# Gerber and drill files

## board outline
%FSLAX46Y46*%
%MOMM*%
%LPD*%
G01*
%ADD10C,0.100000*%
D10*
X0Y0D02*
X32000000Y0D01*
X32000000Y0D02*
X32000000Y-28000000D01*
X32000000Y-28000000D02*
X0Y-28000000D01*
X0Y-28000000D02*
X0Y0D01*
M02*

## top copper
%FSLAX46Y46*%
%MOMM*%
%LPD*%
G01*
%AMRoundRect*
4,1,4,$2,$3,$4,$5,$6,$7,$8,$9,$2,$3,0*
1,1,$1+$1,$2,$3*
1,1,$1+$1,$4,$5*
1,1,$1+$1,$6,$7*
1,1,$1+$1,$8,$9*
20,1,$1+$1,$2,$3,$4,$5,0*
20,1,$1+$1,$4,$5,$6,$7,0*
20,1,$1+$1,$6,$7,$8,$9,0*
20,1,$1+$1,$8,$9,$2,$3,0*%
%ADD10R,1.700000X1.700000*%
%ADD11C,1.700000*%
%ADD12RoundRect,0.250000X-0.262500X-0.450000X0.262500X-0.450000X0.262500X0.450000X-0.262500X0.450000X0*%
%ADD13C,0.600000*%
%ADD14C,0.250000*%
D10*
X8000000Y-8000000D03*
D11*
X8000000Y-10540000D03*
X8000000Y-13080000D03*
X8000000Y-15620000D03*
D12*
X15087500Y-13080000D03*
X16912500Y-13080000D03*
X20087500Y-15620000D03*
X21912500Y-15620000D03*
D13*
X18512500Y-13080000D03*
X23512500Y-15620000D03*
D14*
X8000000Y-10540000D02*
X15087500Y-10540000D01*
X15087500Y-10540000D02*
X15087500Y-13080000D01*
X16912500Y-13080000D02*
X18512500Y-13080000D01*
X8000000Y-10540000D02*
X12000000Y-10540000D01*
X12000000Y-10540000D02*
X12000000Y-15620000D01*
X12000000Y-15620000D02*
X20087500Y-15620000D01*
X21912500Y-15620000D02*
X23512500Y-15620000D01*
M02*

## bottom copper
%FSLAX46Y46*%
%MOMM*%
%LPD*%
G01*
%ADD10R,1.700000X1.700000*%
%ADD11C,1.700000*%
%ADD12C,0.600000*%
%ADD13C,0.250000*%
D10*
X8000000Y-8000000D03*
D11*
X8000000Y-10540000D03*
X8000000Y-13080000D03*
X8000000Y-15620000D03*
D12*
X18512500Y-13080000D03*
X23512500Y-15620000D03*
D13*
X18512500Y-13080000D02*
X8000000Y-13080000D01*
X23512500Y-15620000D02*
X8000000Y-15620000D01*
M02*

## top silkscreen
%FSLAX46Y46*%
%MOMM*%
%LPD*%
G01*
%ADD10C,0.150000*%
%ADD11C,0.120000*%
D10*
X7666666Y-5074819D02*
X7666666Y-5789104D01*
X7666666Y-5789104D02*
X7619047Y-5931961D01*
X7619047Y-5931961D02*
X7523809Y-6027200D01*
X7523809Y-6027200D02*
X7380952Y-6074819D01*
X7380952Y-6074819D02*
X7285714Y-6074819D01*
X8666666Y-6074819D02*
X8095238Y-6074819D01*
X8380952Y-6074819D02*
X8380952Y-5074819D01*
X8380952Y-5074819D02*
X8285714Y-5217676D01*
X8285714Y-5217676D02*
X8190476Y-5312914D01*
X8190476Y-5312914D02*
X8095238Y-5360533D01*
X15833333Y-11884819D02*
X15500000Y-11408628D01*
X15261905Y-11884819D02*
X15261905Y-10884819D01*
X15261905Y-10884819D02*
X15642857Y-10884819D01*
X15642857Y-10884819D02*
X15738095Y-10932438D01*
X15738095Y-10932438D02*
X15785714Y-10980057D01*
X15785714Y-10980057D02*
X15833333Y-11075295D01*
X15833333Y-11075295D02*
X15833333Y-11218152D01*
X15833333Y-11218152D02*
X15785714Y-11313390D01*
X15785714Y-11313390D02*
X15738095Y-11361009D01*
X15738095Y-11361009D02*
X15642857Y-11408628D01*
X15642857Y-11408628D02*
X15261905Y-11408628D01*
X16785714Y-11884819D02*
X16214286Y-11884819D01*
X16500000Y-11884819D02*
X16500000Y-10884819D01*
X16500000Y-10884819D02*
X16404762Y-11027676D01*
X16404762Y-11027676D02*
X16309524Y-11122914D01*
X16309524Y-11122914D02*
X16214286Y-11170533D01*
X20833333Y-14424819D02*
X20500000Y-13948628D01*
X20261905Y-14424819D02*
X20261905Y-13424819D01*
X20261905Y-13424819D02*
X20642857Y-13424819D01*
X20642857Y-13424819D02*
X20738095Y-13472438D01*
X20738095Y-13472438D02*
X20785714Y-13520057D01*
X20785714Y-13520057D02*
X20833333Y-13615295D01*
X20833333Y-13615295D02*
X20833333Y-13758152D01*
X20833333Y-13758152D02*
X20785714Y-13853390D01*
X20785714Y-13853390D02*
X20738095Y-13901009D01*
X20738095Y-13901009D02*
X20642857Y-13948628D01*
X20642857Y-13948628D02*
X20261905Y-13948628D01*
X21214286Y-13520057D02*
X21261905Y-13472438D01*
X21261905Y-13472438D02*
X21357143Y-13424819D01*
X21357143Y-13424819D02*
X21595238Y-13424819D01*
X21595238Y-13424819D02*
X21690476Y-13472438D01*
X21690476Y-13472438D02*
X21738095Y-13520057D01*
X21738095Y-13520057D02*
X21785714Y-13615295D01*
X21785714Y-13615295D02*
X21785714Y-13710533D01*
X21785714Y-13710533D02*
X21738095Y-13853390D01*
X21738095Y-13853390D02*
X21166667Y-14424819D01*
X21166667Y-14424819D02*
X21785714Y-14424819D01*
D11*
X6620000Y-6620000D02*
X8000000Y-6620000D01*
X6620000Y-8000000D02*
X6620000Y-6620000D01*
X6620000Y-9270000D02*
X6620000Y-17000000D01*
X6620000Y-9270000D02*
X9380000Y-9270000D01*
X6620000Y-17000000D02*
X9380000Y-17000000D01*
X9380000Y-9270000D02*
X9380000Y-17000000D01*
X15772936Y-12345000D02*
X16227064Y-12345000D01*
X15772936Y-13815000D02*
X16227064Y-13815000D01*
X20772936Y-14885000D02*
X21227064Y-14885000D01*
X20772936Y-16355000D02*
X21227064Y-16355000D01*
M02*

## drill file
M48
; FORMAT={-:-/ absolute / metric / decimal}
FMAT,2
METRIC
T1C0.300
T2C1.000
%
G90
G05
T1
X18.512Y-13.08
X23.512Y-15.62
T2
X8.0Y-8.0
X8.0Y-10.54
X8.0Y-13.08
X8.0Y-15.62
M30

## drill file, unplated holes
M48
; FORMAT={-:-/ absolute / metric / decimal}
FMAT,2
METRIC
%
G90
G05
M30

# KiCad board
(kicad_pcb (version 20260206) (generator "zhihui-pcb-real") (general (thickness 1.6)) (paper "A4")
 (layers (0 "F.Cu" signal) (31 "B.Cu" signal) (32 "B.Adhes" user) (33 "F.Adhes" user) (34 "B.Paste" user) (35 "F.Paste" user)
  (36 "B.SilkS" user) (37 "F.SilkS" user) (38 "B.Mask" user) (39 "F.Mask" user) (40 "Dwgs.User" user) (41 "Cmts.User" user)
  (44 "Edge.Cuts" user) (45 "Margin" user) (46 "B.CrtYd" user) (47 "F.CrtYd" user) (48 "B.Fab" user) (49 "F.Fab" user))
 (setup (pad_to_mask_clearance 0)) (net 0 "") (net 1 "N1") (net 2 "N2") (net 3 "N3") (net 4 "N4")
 (gr_line (start 0 0) (end 32 0) (stroke (width 0.1) (type default)) (layer "Edge.Cuts"))
 (gr_line (start 32 0) (end 32 28) (stroke (width 0.1) (type default)) (layer "Edge.Cuts"))
 (gr_line (start 32 28) (end 0 28) (stroke (width 0.1) (type default)) (layer "Edge.Cuts"))
 (gr_line (start 0 28) (end 0 0) (stroke (width 0.1) (type default)) (layer "Edge.Cuts"))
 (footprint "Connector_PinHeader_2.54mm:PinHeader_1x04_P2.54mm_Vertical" (layer "F.Cu")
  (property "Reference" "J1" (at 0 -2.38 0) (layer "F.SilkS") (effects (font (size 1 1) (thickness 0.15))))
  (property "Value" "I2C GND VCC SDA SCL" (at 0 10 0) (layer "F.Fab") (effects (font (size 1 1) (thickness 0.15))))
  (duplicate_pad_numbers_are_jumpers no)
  (fp_line (start -1.38 -1.38) (end 0 -1.38) (stroke (width 0.12) (type solid)) (layer "F.SilkS"))
  (fp_line (start -1.38 0) (end -1.38 -1.38) (stroke (width 0.12) (type solid)) (layer "F.SilkS"))
  (fp_line (start -1.38 1.27) (end -1.38 9) (stroke (width 0.12) (type solid)) (layer "F.SilkS"))
  (fp_line (start -1.38 1.27) (end 1.38 1.27) (stroke (width 0.12) (type solid)) (layer "F.SilkS"))
  (fp_line (start -1.38 9) (end 1.38 9) (stroke (width 0.12) (type solid)) (layer "F.SilkS"))
  (fp_line (start 1.38 1.27) (end 1.38 9) (stroke (width 0.12) (type solid)) (layer "F.SilkS"))
  (pad "1" thru_hole rect (at 0 0) (size 1.7 1.7) (drill 1) (layers "*.Cu" "*.Mask") (remove_unused_layers no) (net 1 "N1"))
  (pad "2" thru_hole circle (at 0 2.54) (size 1.7 1.7) (drill 1) (layers "*.Cu" "*.Mask") (remove_unused_layers no) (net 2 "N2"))
  (pad "3" thru_hole circle (at 0 5.08) (size 1.7 1.7) (drill 1) (layers "*.Cu" "*.Mask") (remove_unused_layers no) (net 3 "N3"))
  (pad "4" thru_hole circle (at 0 7.62) (size 1.7 1.7) (drill 1) (layers "*.Cu" "*.Mask") (remove_unused_layers no) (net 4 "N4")) (at 8 8 0))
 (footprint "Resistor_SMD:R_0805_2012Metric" (layer "F.Cu")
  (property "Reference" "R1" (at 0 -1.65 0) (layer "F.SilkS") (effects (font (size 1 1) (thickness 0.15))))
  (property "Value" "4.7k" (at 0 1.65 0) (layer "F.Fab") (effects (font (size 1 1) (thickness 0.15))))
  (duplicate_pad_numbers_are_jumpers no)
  (fp_line (start -0.227064 -0.735) (end 0.227064 -0.735) (stroke (width 0.12) (type solid)) (layer "F.SilkS"))
  (fp_line (start -0.227064 0.735) (end 0.227064 0.735) (stroke (width 0.12) (type solid)) (layer "F.SilkS"))
  (pad "1" smd roundrect (at -0.9125 0) (size 1.025 1.4) (layers "F.Cu" "F.Mask" "F.Paste") (roundrect_rratio 0.243902) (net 2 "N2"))
  (pad "2" smd roundrect (at 0.9125 0) (size 1.025 1.4) (layers "F.Cu" "F.Mask" "F.Paste") (roundrect_rratio 0.243902) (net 3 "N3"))
  (at 16 13.08 0))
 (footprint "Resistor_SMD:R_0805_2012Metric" (layer "F.Cu")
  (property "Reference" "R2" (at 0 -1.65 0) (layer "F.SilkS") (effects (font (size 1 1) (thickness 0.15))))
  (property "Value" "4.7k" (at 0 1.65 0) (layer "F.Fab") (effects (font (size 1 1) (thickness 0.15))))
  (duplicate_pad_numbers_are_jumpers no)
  (fp_line (start -0.227064 -0.735) (end 0.227064 -0.735) (stroke (width 0.12) (type solid)) (layer "F.SilkS"))
  (fp_line (start -0.227064 0.735) (end 0.227064 0.735) (stroke (width 0.12) (type solid)) (layer "F.SilkS"))
  (pad "1" smd roundrect (at -0.9125 0) (size 1.025 1.4) (layers "F.Cu" "F.Mask" "F.Paste") (roundrect_rratio 0.243902) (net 2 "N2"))
  (pad "2" smd roundrect (at 0.9125 0) (size 1.025 1.4) (layers "F.Cu" "F.Mask" "F.Paste") (roundrect_rratio 0.243902) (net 4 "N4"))
  (at 21 15.62 0))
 (segment (start 8 10.54) (end 15.0875 10.54) (width 0.25) (layer "F.Cu") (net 2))
 (segment (start 15.0875 10.54) (end 15.0875 13.08) (width 0.25) (layer "F.Cu") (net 2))
 (segment (start 16.9125 13.08) (end 18.5125 13.08) (width 0.25) (layer "F.Cu") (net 3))
 (segment (start 18.5125 13.08) (end 8 13.08) (width 0.25) (layer "B.Cu") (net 3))
 (segment (start 8 10.54) (end 12 10.54) (width 0.25) (layer "F.Cu") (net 2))
 (segment (start 12 10.54) (end 12 15.62) (width 0.25) (layer "F.Cu") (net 2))
 (segment (start 12 15.62) (end 20.0875 15.62) (width 0.25) (layer "F.Cu") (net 2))
 (segment (start 21.9125 15.62) (end 23.5125 15.62) (width 0.25) (layer "F.Cu") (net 4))
 (segment (start 23.5125 15.62) (end 8 15.62) (width 0.25) (layer "B.Cu") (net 4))
 (via (at 18.5125 13.08) (size 0.6) (drill 0.3) (layers "F.Cu" "B.Cu") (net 3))
 (via (at 23.5125 15.62) (size 0.6) (drill 0.3) (layers "F.Cu" "B.Cu") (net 4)))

